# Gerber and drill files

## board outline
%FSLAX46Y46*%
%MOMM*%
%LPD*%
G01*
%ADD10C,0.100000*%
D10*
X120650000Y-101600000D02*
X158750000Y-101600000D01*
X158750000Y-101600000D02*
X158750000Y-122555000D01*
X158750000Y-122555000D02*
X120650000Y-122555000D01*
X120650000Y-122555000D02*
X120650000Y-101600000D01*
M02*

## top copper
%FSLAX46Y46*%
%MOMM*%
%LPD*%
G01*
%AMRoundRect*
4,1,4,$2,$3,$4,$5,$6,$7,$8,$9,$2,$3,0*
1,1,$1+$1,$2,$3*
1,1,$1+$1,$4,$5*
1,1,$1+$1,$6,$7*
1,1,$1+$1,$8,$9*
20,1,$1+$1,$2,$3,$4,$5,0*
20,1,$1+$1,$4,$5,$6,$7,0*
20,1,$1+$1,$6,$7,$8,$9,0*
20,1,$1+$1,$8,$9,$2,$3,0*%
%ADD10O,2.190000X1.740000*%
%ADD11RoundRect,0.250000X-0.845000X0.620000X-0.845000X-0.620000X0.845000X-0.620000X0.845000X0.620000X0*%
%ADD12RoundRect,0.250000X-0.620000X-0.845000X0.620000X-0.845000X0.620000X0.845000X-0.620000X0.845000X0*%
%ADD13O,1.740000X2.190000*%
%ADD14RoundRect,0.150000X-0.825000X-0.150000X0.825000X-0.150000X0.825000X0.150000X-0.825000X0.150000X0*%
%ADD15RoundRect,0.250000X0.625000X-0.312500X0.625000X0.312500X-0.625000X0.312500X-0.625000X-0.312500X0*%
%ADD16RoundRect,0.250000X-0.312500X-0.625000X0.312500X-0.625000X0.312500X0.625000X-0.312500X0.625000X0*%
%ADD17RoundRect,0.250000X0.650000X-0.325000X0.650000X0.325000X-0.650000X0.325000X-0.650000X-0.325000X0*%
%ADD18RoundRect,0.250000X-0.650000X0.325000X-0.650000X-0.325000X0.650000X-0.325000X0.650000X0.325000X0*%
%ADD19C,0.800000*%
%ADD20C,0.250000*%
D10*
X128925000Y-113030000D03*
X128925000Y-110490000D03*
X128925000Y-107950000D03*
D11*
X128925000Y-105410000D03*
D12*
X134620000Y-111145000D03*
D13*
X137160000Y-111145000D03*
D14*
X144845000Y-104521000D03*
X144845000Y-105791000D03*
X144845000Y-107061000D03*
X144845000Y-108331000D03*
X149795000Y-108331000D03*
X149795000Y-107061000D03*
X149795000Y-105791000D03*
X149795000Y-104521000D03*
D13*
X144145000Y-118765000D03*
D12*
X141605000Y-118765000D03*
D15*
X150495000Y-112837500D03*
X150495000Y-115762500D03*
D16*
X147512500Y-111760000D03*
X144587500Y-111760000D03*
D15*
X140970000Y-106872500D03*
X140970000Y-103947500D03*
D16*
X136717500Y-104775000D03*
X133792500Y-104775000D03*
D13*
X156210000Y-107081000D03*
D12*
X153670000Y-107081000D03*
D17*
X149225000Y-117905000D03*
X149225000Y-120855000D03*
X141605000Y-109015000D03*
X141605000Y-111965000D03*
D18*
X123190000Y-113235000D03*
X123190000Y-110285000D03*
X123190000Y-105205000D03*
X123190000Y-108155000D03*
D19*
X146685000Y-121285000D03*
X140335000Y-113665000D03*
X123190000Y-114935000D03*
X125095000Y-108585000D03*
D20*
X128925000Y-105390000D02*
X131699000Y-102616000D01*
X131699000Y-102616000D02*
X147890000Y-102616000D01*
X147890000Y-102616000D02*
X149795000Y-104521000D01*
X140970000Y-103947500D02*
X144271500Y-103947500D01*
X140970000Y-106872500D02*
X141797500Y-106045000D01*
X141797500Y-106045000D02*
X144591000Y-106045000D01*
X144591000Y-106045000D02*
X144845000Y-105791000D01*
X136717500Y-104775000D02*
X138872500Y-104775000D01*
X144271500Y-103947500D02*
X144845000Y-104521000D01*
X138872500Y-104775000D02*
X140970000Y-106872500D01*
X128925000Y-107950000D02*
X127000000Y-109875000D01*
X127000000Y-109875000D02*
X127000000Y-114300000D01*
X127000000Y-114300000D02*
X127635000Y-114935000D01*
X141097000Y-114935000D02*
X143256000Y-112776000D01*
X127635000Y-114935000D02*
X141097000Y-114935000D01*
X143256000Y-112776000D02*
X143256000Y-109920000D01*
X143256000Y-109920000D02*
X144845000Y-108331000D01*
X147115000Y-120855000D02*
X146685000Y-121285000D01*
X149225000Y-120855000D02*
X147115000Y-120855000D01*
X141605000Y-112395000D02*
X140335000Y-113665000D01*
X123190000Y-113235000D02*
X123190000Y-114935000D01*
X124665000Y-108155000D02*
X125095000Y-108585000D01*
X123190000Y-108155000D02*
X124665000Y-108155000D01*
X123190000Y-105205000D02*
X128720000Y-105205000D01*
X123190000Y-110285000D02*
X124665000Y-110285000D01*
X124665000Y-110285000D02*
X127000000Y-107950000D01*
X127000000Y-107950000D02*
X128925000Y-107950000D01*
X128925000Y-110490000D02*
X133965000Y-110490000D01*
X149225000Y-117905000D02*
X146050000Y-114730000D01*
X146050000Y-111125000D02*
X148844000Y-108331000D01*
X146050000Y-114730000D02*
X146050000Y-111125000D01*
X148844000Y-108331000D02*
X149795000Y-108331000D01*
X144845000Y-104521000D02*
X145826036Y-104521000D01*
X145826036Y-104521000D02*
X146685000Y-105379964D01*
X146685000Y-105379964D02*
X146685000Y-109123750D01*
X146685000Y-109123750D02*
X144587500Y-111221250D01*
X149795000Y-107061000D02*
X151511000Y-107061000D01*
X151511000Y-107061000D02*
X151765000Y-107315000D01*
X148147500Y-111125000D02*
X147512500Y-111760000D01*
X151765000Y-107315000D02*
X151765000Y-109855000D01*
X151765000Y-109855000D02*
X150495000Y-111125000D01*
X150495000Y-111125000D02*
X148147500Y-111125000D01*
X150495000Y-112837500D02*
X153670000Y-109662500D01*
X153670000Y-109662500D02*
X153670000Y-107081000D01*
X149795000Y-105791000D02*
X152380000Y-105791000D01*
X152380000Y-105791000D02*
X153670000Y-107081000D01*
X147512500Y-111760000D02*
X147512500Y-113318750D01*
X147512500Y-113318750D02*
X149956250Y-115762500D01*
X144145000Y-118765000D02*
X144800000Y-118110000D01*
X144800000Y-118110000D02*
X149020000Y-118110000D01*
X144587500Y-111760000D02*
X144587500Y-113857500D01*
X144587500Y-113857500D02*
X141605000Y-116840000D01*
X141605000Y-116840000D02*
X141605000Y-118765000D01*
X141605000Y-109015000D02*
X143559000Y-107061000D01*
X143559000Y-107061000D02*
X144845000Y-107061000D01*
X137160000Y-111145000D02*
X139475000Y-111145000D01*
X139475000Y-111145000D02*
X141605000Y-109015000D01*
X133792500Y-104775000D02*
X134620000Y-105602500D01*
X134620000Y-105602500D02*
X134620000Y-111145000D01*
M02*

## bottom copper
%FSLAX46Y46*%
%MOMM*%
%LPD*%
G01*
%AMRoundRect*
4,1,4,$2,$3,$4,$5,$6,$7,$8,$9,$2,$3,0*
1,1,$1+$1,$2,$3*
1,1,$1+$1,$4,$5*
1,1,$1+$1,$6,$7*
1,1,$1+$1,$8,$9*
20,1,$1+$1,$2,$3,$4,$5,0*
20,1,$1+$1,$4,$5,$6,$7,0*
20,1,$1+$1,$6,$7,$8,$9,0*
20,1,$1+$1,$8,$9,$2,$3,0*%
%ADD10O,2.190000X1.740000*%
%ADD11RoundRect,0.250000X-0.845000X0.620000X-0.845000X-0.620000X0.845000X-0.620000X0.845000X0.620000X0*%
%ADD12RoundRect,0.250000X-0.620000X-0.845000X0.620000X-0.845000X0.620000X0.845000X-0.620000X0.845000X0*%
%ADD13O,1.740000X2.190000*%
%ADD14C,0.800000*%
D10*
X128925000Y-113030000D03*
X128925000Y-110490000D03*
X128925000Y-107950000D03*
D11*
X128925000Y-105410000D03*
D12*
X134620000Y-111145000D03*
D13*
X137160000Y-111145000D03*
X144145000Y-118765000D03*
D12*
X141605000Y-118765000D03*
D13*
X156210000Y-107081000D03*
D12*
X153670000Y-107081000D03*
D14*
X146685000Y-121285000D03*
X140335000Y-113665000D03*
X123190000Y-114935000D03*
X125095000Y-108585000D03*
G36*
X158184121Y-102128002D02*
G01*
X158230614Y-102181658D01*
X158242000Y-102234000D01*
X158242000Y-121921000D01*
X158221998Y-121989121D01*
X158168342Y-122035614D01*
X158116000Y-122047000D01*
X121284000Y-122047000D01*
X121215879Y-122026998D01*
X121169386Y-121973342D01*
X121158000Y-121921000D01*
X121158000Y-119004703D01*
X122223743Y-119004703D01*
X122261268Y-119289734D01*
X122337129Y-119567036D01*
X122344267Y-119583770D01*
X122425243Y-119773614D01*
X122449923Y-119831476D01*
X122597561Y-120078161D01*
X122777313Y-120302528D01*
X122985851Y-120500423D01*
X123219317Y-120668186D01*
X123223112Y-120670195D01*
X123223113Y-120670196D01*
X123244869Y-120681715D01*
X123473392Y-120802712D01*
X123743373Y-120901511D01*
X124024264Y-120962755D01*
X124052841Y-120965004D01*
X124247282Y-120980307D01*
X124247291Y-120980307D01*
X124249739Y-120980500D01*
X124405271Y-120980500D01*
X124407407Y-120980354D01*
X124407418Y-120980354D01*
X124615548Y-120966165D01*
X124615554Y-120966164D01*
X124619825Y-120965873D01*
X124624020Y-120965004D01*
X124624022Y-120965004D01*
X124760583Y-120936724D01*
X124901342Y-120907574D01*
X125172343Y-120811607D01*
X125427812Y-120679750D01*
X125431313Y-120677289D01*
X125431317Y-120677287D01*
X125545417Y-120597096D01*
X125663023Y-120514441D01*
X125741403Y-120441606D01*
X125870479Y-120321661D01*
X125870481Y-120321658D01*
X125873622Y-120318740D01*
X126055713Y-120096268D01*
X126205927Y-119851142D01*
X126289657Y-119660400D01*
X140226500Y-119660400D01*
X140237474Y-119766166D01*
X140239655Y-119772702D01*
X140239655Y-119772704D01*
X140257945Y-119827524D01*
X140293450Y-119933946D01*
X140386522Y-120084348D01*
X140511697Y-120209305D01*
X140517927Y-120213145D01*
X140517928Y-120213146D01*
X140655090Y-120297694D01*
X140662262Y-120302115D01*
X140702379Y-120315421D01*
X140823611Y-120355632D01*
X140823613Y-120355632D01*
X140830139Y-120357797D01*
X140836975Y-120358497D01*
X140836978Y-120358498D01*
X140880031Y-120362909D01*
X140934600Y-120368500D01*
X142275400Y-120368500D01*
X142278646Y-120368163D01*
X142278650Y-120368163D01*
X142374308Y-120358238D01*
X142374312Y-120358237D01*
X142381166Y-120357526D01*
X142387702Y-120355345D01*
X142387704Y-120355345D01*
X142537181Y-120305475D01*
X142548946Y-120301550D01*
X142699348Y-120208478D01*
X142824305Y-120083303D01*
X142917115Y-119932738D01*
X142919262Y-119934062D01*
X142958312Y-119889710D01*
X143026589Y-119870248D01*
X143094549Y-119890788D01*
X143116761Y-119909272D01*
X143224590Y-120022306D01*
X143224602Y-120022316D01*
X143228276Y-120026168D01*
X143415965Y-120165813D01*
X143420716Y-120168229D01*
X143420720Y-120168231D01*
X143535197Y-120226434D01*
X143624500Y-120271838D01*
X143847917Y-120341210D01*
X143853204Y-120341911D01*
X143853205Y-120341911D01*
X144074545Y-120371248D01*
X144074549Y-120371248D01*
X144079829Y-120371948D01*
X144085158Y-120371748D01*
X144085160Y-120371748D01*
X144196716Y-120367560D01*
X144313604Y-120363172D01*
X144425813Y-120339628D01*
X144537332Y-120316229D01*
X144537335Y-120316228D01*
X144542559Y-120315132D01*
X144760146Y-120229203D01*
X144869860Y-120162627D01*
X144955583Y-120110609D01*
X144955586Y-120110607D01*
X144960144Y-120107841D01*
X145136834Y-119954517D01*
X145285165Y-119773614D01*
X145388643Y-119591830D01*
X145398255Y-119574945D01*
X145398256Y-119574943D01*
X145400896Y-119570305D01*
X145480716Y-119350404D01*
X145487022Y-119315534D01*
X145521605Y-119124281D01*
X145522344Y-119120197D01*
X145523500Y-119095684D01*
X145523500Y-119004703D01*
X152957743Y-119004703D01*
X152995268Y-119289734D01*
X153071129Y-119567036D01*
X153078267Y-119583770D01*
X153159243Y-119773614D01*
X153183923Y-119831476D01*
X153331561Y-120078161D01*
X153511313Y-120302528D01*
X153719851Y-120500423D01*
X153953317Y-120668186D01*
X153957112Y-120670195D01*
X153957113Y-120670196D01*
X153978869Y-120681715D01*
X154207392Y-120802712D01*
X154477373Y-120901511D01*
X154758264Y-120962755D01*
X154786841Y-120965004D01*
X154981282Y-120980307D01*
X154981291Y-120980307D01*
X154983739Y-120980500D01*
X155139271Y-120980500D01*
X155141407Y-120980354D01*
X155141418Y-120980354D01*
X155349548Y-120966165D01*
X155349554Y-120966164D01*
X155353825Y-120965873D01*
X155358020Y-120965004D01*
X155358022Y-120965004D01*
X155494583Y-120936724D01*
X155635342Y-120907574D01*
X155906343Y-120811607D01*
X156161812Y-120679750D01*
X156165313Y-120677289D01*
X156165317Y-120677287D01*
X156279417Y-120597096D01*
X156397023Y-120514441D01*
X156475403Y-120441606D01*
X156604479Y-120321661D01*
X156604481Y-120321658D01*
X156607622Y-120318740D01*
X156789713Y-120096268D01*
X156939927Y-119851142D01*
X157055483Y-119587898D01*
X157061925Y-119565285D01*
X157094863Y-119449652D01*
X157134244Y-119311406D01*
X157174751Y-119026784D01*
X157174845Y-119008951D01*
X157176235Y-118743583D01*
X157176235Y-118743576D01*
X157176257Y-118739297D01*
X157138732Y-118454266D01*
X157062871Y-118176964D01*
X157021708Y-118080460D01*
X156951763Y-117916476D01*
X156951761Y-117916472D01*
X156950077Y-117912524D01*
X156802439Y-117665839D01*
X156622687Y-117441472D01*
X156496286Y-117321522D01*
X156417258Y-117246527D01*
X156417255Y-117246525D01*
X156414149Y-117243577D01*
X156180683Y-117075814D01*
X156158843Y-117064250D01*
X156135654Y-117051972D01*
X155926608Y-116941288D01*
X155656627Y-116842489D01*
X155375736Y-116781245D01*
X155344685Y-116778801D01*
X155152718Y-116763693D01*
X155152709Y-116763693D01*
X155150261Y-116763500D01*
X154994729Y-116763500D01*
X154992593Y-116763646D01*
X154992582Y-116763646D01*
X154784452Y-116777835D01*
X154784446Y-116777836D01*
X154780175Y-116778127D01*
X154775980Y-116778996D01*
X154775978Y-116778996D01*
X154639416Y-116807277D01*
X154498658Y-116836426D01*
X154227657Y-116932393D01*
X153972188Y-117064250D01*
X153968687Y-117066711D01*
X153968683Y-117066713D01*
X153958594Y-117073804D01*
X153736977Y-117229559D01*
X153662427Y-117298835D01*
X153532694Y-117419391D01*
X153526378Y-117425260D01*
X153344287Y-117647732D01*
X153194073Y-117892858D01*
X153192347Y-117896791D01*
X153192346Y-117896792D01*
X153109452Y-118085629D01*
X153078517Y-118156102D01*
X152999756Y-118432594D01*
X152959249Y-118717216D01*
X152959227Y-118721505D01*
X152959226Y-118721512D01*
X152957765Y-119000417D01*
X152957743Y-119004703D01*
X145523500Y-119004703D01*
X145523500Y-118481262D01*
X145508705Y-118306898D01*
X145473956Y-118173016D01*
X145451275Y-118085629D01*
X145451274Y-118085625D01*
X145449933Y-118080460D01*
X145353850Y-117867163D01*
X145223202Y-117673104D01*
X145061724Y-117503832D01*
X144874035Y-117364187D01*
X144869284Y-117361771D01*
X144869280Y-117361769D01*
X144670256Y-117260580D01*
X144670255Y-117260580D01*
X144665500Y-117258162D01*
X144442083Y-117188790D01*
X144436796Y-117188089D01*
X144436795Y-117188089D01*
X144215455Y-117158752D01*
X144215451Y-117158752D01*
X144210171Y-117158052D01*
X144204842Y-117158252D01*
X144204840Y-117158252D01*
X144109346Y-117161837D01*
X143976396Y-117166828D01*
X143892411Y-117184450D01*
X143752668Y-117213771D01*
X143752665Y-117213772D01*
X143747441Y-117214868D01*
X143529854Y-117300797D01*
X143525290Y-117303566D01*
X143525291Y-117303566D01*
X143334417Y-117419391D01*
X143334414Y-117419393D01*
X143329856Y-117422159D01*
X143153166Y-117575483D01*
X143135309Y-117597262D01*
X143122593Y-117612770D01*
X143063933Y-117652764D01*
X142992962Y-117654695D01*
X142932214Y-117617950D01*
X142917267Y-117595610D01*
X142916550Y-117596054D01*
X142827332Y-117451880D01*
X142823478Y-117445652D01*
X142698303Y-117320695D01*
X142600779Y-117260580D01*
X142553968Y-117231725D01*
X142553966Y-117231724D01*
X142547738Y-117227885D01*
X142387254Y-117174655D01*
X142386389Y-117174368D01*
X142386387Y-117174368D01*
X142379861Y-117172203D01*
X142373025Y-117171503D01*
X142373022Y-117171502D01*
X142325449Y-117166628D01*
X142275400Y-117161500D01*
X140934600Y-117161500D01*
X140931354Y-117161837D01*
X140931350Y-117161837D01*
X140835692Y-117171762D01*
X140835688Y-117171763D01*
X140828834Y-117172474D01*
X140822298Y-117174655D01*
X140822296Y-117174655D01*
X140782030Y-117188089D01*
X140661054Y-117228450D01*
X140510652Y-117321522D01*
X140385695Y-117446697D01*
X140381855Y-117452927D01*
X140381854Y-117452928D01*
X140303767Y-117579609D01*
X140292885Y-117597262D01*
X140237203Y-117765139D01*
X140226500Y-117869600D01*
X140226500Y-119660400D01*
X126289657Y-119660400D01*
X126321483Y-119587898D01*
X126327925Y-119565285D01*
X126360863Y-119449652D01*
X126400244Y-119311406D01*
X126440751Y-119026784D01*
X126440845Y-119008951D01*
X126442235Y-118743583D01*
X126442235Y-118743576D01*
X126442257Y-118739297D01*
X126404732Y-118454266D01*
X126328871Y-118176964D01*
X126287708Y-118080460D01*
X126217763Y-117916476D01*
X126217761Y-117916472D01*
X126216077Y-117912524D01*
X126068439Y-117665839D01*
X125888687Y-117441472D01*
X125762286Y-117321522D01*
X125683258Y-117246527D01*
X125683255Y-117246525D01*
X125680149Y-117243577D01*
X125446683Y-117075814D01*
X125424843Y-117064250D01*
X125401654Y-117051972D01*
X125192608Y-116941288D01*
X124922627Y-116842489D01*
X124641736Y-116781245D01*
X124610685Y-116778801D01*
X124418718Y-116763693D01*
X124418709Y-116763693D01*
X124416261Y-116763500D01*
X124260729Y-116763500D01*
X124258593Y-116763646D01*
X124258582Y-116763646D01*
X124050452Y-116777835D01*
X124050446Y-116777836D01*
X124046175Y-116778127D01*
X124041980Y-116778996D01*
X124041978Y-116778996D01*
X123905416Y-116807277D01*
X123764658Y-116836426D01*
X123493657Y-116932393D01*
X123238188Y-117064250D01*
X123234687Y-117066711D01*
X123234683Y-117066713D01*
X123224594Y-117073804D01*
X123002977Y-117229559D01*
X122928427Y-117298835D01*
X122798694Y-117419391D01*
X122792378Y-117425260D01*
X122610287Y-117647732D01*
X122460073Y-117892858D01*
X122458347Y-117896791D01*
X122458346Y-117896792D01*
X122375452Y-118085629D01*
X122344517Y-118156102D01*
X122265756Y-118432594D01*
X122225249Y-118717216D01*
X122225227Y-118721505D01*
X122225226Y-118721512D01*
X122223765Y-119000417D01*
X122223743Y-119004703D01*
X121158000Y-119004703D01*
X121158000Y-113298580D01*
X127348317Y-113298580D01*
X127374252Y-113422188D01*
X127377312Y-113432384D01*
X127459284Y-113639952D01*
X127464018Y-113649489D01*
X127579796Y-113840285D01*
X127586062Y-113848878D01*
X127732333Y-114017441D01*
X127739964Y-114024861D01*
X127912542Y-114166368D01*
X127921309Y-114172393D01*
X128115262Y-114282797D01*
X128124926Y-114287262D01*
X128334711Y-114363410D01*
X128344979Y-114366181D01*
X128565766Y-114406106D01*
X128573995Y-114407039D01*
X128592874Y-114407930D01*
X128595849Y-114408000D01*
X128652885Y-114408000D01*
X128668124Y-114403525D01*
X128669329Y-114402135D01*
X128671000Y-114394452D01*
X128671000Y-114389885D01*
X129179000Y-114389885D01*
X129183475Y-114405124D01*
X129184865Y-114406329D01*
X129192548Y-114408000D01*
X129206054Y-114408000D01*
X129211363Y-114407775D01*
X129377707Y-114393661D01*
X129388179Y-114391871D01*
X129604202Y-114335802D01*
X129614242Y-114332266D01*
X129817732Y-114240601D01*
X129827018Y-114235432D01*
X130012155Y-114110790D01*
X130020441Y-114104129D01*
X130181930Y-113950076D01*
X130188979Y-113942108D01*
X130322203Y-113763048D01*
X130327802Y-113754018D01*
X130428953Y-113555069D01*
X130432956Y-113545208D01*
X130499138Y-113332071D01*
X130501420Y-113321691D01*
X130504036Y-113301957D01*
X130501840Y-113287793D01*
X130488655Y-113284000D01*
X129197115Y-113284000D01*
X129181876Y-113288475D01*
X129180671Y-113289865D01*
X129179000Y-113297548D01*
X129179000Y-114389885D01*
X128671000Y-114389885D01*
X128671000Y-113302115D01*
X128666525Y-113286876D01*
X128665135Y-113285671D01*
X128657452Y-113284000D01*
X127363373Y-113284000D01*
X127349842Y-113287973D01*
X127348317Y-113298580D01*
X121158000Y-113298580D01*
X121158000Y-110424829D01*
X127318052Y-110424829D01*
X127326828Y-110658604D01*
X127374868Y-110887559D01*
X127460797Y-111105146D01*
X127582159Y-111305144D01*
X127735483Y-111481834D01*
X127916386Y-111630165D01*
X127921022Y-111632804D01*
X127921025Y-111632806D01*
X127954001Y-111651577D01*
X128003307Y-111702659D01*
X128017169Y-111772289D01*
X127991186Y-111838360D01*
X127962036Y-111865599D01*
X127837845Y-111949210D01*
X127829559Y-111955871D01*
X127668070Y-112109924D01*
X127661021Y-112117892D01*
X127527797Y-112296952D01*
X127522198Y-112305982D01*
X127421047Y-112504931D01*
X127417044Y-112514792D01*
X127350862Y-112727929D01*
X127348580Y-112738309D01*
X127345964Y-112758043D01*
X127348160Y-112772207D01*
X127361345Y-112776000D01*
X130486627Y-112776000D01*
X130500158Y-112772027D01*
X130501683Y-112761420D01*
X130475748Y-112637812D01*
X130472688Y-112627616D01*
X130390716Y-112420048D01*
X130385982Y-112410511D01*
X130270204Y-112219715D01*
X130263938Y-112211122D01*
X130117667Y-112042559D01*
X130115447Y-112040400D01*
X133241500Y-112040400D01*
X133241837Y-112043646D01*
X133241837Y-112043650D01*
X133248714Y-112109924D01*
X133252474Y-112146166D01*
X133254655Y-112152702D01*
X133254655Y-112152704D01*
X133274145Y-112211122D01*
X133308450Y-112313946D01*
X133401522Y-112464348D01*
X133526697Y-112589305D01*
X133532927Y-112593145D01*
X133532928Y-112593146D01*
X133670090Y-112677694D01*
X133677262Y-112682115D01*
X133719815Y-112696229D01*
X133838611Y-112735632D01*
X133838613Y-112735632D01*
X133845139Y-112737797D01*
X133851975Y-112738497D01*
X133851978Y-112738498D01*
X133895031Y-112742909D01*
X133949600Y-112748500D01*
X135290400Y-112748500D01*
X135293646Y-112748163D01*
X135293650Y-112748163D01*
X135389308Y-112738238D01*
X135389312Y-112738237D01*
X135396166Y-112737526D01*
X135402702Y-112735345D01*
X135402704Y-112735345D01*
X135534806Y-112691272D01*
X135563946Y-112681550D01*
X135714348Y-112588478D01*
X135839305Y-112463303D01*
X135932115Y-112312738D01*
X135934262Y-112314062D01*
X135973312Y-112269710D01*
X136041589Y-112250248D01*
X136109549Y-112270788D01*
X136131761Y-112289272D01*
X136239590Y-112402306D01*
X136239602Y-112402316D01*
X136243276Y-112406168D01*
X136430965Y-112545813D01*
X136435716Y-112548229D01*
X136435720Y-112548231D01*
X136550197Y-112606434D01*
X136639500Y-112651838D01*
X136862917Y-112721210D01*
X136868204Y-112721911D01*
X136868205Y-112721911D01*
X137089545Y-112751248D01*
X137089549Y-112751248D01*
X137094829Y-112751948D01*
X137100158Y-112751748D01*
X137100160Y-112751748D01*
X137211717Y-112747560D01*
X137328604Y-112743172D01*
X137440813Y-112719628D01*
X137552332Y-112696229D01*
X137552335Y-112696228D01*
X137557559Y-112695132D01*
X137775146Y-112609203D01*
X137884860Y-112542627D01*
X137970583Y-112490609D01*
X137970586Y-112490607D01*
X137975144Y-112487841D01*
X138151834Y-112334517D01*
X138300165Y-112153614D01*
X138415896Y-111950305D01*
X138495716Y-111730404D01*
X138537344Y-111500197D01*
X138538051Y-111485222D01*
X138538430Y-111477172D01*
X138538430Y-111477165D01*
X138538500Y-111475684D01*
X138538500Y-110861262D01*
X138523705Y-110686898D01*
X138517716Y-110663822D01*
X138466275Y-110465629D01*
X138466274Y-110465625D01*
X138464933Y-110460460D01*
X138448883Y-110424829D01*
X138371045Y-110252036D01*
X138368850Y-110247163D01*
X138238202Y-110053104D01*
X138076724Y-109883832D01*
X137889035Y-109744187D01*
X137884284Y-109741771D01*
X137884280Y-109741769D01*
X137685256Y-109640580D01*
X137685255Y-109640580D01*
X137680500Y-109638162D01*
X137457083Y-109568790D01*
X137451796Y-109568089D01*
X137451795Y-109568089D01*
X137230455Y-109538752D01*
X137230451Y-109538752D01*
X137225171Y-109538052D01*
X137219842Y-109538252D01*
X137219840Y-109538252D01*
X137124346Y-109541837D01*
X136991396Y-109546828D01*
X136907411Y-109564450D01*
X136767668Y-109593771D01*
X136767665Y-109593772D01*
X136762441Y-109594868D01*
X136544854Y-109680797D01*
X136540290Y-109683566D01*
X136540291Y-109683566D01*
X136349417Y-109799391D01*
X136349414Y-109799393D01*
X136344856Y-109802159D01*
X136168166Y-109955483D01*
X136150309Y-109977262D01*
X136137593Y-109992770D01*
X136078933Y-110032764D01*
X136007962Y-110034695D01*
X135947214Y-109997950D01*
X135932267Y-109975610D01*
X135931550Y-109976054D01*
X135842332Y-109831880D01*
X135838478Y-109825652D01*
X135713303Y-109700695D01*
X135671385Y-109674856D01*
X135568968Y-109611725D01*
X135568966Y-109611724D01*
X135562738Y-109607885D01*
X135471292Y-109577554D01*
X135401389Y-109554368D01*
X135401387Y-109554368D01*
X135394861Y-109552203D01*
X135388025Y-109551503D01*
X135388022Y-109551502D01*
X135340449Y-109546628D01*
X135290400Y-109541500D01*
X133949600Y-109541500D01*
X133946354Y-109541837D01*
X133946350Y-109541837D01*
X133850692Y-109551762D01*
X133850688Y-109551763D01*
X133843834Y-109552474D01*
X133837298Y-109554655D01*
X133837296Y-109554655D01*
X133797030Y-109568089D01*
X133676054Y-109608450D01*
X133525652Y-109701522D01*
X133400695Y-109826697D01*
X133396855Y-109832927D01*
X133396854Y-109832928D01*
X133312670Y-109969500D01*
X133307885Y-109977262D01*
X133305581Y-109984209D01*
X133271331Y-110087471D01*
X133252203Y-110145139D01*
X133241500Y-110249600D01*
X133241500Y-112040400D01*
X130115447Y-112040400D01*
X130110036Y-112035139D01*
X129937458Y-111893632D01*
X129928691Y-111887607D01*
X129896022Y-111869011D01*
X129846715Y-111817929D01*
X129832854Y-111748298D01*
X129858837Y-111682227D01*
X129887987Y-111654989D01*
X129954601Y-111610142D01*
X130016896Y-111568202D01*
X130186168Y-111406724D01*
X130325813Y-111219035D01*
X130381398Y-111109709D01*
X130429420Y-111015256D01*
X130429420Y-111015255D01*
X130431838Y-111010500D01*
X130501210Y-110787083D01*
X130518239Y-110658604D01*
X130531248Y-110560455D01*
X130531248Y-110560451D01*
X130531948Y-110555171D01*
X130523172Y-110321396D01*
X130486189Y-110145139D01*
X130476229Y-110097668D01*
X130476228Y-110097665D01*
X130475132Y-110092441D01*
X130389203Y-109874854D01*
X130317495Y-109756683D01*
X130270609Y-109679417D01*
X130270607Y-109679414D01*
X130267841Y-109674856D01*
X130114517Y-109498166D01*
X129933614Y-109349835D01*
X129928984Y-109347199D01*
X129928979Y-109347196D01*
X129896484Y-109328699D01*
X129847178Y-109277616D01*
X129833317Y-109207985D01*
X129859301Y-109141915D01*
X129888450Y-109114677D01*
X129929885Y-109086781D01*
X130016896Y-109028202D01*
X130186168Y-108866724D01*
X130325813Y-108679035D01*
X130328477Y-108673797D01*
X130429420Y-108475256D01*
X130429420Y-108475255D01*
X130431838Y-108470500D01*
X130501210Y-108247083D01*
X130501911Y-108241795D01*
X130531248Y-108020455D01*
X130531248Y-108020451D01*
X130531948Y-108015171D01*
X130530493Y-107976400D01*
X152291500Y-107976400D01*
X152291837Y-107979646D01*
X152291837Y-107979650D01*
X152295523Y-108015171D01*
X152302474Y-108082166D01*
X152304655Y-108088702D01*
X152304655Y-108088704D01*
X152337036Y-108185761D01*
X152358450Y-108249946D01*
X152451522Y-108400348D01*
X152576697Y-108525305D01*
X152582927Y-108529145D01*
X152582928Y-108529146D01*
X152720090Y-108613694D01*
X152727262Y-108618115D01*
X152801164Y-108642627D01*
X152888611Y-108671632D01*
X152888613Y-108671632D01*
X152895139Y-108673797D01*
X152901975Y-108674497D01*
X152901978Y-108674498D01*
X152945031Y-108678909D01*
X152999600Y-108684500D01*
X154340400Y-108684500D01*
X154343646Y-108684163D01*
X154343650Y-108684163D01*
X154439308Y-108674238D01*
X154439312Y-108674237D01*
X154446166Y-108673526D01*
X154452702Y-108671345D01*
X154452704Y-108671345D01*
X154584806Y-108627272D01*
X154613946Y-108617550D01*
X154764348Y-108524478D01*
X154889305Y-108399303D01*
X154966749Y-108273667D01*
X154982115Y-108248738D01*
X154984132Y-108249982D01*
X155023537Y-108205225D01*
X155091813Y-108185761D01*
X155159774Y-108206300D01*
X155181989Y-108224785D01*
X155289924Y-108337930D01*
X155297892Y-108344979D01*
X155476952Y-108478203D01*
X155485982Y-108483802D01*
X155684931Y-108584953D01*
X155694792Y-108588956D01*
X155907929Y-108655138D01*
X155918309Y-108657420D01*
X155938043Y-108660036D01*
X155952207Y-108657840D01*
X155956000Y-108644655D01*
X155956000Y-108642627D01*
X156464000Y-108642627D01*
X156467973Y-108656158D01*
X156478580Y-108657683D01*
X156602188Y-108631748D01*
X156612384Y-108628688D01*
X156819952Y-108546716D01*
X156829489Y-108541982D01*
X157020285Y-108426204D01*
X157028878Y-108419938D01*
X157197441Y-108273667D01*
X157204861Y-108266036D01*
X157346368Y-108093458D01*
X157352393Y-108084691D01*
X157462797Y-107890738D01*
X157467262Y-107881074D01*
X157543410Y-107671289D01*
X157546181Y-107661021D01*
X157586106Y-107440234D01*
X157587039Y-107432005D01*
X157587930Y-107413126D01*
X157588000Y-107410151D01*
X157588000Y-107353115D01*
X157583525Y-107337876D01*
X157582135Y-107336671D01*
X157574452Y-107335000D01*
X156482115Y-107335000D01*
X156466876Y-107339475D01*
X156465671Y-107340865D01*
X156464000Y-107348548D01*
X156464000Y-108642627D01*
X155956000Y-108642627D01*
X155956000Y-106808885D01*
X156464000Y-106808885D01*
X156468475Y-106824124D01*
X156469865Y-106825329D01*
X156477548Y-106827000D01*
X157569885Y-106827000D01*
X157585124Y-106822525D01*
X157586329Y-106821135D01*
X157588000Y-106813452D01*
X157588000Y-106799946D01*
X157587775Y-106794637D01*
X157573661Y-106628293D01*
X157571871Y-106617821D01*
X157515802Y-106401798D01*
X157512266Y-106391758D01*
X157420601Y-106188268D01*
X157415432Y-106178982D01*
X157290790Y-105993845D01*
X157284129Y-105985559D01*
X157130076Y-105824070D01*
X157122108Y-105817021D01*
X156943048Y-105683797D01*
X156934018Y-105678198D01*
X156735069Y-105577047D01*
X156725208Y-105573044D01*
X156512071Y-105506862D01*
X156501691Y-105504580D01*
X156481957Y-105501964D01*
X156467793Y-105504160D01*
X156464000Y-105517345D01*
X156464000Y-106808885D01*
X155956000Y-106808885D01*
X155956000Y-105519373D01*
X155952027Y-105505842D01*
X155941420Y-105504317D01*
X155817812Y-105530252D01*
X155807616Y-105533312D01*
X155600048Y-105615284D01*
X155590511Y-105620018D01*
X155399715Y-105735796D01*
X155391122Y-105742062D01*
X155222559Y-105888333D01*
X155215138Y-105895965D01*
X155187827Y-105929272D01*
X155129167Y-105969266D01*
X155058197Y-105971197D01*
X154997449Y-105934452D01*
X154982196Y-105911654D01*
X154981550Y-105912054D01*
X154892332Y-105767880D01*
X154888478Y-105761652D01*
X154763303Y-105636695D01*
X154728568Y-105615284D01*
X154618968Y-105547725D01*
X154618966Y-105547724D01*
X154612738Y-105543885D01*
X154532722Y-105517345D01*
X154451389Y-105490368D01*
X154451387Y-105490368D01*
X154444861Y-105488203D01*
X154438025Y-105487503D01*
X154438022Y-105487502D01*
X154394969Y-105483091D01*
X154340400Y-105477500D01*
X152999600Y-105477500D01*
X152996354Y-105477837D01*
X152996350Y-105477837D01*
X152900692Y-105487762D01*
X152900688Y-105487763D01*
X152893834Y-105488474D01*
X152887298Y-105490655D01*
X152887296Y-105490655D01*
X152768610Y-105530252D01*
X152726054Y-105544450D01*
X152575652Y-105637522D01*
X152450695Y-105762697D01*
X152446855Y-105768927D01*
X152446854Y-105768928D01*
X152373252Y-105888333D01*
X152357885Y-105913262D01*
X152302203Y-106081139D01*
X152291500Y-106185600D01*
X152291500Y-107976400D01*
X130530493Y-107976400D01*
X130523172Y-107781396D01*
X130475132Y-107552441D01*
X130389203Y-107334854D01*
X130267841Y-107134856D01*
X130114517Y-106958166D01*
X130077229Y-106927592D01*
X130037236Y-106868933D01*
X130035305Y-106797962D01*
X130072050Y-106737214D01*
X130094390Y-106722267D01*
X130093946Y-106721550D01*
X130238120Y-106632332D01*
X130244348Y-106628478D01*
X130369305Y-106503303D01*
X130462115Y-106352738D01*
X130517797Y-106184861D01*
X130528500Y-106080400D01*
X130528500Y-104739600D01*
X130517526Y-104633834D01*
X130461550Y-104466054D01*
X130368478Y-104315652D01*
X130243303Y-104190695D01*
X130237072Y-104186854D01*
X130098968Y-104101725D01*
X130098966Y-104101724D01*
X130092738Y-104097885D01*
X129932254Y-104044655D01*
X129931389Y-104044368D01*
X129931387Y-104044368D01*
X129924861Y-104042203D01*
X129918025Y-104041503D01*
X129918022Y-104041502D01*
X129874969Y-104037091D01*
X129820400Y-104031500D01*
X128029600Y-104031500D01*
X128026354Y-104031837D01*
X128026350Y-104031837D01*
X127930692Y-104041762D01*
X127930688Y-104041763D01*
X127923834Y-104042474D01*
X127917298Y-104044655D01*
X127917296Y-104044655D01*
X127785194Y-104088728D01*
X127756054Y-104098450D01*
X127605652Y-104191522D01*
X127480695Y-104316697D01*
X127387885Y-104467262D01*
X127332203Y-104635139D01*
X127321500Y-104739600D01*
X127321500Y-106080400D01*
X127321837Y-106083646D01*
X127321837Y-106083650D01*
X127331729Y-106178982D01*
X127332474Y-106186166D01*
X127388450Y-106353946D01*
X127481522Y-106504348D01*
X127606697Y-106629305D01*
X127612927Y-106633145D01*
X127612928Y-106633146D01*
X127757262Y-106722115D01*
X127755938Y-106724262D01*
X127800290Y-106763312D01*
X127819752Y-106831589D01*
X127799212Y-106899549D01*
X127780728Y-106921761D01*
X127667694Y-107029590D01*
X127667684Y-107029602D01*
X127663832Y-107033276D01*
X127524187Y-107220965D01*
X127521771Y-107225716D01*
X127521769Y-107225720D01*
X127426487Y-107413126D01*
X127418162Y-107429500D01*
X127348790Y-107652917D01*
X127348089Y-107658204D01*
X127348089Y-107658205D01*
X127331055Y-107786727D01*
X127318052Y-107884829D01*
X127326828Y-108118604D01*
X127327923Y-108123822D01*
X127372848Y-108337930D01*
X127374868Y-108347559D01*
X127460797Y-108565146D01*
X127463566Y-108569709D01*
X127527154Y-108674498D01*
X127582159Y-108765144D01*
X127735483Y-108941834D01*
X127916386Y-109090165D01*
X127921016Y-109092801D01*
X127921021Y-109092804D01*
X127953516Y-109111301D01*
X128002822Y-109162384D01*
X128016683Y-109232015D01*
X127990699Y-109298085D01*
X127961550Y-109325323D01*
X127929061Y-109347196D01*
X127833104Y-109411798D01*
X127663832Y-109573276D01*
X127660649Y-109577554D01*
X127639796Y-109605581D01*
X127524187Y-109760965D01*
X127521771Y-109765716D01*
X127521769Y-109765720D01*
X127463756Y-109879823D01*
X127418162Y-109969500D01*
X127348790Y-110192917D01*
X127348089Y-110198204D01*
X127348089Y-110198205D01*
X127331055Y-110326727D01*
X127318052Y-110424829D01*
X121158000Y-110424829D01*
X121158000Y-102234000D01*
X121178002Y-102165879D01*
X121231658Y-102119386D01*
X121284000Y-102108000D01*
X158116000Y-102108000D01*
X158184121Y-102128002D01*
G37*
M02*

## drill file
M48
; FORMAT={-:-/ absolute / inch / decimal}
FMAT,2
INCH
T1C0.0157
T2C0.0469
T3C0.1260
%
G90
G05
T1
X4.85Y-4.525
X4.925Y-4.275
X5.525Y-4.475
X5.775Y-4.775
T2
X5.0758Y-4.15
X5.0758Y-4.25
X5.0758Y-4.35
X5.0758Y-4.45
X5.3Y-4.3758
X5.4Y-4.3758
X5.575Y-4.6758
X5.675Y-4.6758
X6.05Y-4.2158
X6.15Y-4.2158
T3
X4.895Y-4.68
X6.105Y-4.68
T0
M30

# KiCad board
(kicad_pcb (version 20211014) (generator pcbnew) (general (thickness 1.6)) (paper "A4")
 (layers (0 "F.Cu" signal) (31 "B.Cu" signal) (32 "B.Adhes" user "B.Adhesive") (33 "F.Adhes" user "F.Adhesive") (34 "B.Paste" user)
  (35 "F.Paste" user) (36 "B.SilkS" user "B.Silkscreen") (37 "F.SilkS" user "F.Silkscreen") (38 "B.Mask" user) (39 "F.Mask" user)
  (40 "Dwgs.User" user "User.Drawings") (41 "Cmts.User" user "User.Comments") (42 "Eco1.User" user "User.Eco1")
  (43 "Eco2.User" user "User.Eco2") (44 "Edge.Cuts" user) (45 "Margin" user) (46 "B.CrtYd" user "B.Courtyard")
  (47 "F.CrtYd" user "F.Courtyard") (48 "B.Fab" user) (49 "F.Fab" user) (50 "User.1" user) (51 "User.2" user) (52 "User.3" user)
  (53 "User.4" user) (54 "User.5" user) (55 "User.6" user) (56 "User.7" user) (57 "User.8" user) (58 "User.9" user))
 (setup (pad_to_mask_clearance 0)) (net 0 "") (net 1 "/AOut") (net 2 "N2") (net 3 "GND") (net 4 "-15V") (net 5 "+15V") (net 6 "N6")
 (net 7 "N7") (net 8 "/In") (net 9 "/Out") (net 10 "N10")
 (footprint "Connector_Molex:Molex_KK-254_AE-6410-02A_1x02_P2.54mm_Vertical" (layer "F.Cu") (at 141.605 118.765)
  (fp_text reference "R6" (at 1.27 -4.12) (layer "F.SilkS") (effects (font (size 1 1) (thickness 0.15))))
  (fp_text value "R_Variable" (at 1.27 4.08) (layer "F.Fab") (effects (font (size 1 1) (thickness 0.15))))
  (pad "1" thru_hole roundrect (at 0 0) (size 1.74 2.19) (drill 1.19) (layers *.Cu *.Mask) (roundrect_rratio 0.1436781609) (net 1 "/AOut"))
  (pad "2" thru_hole oval (at 2.54 0) (size 1.74 2.19) (drill 1.19) (layers *.Cu *.Mask) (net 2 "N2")))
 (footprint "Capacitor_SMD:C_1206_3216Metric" (layer "F.Cu") (at 149.225 119.38 90)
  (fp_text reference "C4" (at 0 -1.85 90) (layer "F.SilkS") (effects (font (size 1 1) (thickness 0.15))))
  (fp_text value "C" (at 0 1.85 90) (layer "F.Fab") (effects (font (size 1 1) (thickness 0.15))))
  (pad "1" smd roundrect (at -1.475 0 90) (size 1.15 1.8) (layers "F.Cu" "F.Paste" "F.Mask") (roundrect_rratio 0.2173913043) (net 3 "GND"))
  (pad "2" smd roundrect (at 1.475 0 90) (size 1.15 1.8) (layers "F.Cu" "F.Paste" "F.Mask") (roundrect_rratio 0.2173913043) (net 2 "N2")))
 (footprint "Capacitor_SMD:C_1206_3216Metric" (layer "F.Cu") (at 123.19 111.76 -90)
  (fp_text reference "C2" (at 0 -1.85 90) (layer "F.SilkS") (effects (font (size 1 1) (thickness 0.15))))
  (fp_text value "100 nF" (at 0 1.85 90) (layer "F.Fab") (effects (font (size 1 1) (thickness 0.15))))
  (pad "1" smd roundrect (at -1.475 0 270) (size 1.15 1.8) (layers "F.Cu" "F.Paste" "F.Mask") (roundrect_rratio 0.2173913043) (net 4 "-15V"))
  (pad "2" smd roundrect (at 1.475 0 270) (size 1.15 1.8) (layers "F.Cu" "F.Paste" "F.Mask") (roundrect_rratio 0.2173913043) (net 3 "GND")))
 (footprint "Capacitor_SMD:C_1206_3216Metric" (layer "F.Cu") (at 123.19 106.68 -90)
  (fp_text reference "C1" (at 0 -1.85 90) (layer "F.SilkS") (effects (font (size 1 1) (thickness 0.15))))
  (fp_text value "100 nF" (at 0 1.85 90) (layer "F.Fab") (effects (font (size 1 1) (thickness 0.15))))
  (pad "1" smd roundrect (at -1.475 0 270) (size 1.15 1.8) (layers "F.Cu" "F.Paste" "F.Mask") (roundrect_rratio 0.2173913043) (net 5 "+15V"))
  (pad "2" smd roundrect (at 1.475 0 270) (size 1.15 1.8) (layers "F.Cu" "F.Paste" "F.Mask") (roundrect_rratio 0.2173913043) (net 3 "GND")))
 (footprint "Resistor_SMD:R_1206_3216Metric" (layer "F.Cu") (at 146.05 111.76)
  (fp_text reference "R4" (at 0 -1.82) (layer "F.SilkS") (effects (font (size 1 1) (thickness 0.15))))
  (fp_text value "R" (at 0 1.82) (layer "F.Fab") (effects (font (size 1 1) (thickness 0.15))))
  (pad "1" smd roundrect (at -1.4625 0) (size 1.125 1.75) (layers "F.Cu" "F.Paste" "F.Mask") (roundrect_rratio 0.2222222222) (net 1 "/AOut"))
  (pad "2" smd roundrect (at 1.4625 0) (size 1.125 1.75) (layers "F.Cu" "F.Paste" "F.Mask") (roundrect_rratio 0.2222222222) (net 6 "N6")))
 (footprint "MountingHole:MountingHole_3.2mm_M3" (layer "F.Cu") (at 124.333 118.872)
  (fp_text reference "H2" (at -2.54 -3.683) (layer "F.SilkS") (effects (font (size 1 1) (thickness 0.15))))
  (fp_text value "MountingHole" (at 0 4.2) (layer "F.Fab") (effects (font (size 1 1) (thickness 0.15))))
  (pad "" np_thru_hole circle (at 0 0) (size 3.2 3.2) (drill 3.2) (layers *.Cu *.Mask)))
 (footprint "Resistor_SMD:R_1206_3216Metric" (layer "F.Cu") (at 140.97 105.41 90)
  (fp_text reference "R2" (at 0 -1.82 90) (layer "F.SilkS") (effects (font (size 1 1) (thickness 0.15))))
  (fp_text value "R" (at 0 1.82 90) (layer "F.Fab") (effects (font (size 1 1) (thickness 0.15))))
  (pad "1" smd roundrect (at -1.4625 0 90) (size 1.125 1.75) (layers "F.Cu" "F.Paste" "F.Mask") (roundrect_rratio 0.2222222222) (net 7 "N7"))
  (pad "2" smd roundrect (at 1.4625 0 90) (size 1.125 1.75) (layers "F.Cu" "F.Paste" "F.Mask") (roundrect_rratio 0.2222222222)
   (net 1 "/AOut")))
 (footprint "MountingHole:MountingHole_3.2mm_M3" (layer "F.Cu") (at 155.067 118.872)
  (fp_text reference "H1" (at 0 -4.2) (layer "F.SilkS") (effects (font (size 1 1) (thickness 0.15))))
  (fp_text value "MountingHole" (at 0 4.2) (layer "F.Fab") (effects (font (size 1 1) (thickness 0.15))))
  (pad "" np_thru_hole circle (at 0 0) (size 3.2 3.2) (drill 3.2) (layers *.Cu *.Mask)))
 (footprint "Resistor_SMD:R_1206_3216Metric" (layer "F.Cu") (at 135.255 104.775)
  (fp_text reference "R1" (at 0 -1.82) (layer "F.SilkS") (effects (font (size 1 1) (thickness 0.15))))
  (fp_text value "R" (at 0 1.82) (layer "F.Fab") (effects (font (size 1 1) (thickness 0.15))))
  (pad "1" smd roundrect (at -1.4625 0) (size 1.125 1.75) (layers "F.Cu" "F.Paste" "F.Mask") (roundrect_rratio 0.2222222222) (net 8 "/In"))
  (pad "2" smd roundrect (at 1.4625 0) (size 1.125 1.75) (layers "F.Cu" "F.Paste" "F.Mask") (roundrect_rratio 0.2222222222) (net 7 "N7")))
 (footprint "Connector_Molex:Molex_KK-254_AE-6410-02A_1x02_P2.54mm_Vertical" (layer "F.Cu") (at 153.67 107.081)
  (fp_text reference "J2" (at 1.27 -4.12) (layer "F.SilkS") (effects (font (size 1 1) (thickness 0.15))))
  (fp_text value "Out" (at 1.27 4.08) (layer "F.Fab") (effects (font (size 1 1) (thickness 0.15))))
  (pad "1" thru_hole roundrect (at 0 0) (size 1.74 2.19) (drill 1.19) (layers *.Cu *.Mask) (roundrect_rratio 0.1436781609) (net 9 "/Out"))
  (pad "2" thru_hole oval (at 2.54 0) (size 1.74 2.19) (drill 1.19) (layers *.Cu *.Mask) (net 3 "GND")))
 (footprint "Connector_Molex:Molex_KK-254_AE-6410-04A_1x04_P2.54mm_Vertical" (layer "F.Cu") (at 128.925 105.41 -90)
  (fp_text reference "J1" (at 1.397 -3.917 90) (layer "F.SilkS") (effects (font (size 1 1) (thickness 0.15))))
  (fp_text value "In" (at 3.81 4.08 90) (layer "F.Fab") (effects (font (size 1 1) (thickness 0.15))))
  (pad "1" thru_hole roundrect (at 0 0 270) (size 1.74 2.19) (drill 1.19) (layers *.Cu *.Mask) (roundrect_rratio 0.1436781609)
   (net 5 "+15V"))
  (pad "2" thru_hole oval (at 2.54 0 270) (size 1.74 2.19) (drill 1.19) (layers *.Cu *.Mask) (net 4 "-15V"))
  (pad "3" thru_hole oval (at 5.08 0 270) (size 1.74 2.19) (drill 1.19) (layers *.Cu *.Mask) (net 8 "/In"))
  (pad "4" thru_hole oval (at 7.62 0 270) (size 1.74 2.19) (drill 1.19) (layers *.Cu *.Mask) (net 3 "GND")))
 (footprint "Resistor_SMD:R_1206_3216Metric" (layer "F.Cu") (at 150.495 114.3 90)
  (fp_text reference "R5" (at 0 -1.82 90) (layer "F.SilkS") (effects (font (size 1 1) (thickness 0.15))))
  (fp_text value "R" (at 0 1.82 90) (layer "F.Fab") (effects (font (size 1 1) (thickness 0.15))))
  (pad "1" smd roundrect (at -1.4625 0 90) (size 1.125 1.75) (layers "F.Cu" "F.Paste" "F.Mask") (roundrect_rratio 0.2222222222) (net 6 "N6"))
  (pad "2" smd roundrect (at 1.4625 0 90) (size 1.125 1.75) (layers "F.Cu" "F.Paste" "F.Mask") (roundrect_rratio 0.2222222222)
   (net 9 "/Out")))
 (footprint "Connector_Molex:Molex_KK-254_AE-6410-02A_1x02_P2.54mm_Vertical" (layer "F.Cu") (at 134.62 111.145)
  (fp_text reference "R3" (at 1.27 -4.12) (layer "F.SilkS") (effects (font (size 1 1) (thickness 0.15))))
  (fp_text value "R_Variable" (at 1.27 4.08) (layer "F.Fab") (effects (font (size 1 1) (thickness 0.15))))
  (pad "1" thru_hole roundrect (at 0 0) (size 1.74 2.19) (drill 1.19) (layers *.Cu *.Mask) (roundrect_rratio 0.1436781609) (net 8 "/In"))
  (pad "2" thru_hole oval (at 2.54 0) (size 1.74 2.19) (drill 1.19) (layers *.Cu *.Mask) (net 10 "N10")))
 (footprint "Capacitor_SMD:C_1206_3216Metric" (layer "F.Cu") (at 141.605 110.49 90)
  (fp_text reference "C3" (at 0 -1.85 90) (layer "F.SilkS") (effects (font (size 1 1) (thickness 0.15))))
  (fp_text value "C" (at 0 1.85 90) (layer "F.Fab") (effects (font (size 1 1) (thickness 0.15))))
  (pad "1" smd roundrect (at -1.475 0 90) (size 1.15 1.8) (layers "F.Cu" "F.Paste" "F.Mask") (roundrect_rratio 0.2173913043) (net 3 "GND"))
  (pad "2" smd roundrect (at 1.475 0 90) (size 1.15 1.8) (layers "F.Cu" "F.Paste" "F.Mask") (roundrect_rratio 0.2173913043) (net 10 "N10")))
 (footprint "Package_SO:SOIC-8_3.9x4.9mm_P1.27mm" (layer "F.Cu") (at 147.32 106.426)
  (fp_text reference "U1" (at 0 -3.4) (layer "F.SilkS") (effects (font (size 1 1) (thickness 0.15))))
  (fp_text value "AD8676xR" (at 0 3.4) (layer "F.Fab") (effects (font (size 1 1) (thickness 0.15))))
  (pad "1" smd roundrect (at -2.475 -1.905) (size 1.95 0.6) (layers "F.Cu" "F.Paste" "F.Mask") (roundrect_rratio 0.25) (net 1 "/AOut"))
  (pad "2" smd roundrect (at -2.475 -0.635) (size 1.95 0.6) (layers "F.Cu" "F.Paste" "F.Mask") (roundrect_rratio 0.25) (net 7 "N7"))
  (pad "3" smd roundrect (at -2.475 0.635) (size 1.95 0.6) (layers "F.Cu" "F.Paste" "F.Mask") (roundrect_rratio 0.25) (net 10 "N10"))
  (pad "4" smd roundrect (at -2.475 1.905) (size 1.95 0.6) (layers "F.Cu" "F.Paste" "F.Mask") (roundrect_rratio 0.25) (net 4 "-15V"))
  (pad "5" smd roundrect (at 2.475 1.905) (size 1.95 0.6) (layers "F.Cu" "F.Paste" "F.Mask") (roundrect_rratio 0.25) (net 2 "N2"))
  (pad "6" smd roundrect (at 2.475 0.635) (size 1.95 0.6) (layers "F.Cu" "F.Paste" "F.Mask") (roundrect_rratio 0.25) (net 6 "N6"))
  (pad "7" smd roundrect (at 2.475 -0.635) (size 1.95 0.6) (layers "F.Cu" "F.Paste" "F.Mask") (roundrect_rratio 0.25) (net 9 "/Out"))
  (pad "8" smd roundrect (at 2.475 -1.905) (size 1.95 0.6) (layers "F.Cu" "F.Paste" "F.Mask") (roundrect_rratio 0.25) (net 5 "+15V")))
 (gr_rect (start 120.65 101.6) (end 158.75 122.555) (layer "Edge.Cuts") (width 0.1) (fill none))
 (segment (start 131.699 102.616) (end 147.89 102.616) (width 0.25) (layer "F.Cu") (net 5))
 (segment (start 123.19 105.205) (end 128.72 105.205) (width 0.25) (layer "F.Cu") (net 5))
 (segment (start 128.925 105.39) (end 131.699 102.616) (width 0.25) (layer "F.Cu") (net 5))
 (segment (start 147.89 102.616) (end 149.795 104.521) (width 0.25) (layer "F.Cu") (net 5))
 (segment (start 123.19 113.235) (end 123.19 114.935) (width 0.25) (layer "F.Cu") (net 3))
 (segment (start 149.225 120.855) (end 147.115 120.855) (width 0.25) (layer "F.Cu") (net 3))
 (segment (start 141.605 112.395) (end 140.335 113.665) (width 0.25) (layer "F.Cu") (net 3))
 (segment (start 124.665 108.155) (end 125.095 108.585) (width 0.25) (layer "F.Cu") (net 3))
 (segment (start 147.115 120.855) (end 146.685 121.285) (width 0.25) (layer "F.Cu") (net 3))
 (segment (start 123.19 108.155) (end 124.665 108.155) (width 0.25) (layer "F.Cu") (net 3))
 (via (at 140.335 113.665) (size 0.8) (drill 0.4) (layers "F.Cu" "B.Cu") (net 3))
 (via (at 125.095 108.585) (size 0.8) (drill 0.4) (layers "F.Cu" "B.Cu") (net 3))
 (via (at 123.19 114.935) (size 0.8) (drill 0.4) (layers "F.Cu" "B.Cu") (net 3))
 (via (at 146.685 121.285) (size 0.8) (drill 0.4) (layers "F.Cu" "B.Cu") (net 3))
 (segment (start 123.19 110.285) (end 124.665 110.285) (width 0.25) (layer "F.Cu") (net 4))
 (segment (start 127.635 114.935) (end 141.097 114.935) (width 0.25) (layer "F.Cu") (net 4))
 (segment (start 143.256 112.776) (end 143.256 109.92) (width 0.25) (layer "F.Cu") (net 4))
 (segment (start 127 107.95) (end 128.925 107.95) (width 0.25) (layer "F.Cu") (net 4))
 (segment (start 143.256 109.92) (end 144.845 108.331) (width 0.25) (layer "F.Cu") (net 4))
 (segment (start 127 114.3) (end 127.635 114.935) (width 0.25) (layer "F.Cu") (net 4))
 (segment (start 127 109.875) (end 127 114.3) (width 0.25) (layer "F.Cu") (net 4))
 (segment (start 124.665 110.285) (end 127 107.95) (width 0.25) (layer "F.Cu") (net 4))
 (segment (start 128.925 107.95) (end 127 109.875) (width 0.25) (layer "F.Cu") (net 4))
 (segment (start 141.097 114.935) (end 143.256 112.776) (width 0.25) (layer "F.Cu") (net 4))
 (segment (start 133.7925 104.775) (end 134.62 105.6025) (width 0.25) (layer "F.Cu") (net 8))
 (segment (start 128.925 110.49) (end 133.965 110.49) (width 0.25) (layer "F.Cu") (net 8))
 (segment (start 134.62 105.6025) (end 134.62 111.145) (width 0.25) (layer "F.Cu") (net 8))
 (segment (start 150.495 112.8375) (end 153.67 109.6625) (width 0.25) (layer "F.Cu") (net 9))
 (segment (start 153.67 109.6625) (end 153.67 107.081) (width 0.25) (layer "F.Cu") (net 9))
 (segment (start 152.38 105.791) (end 153.67 107.081) (width 0.25) (layer "F.Cu") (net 9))
 (segment (start 149.795 105.791) (end 152.38 105.791) (width 0.25) (layer "F.Cu") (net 9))
 (segment (start 136.7175 104.775) (end 138.8725 104.775) (width 0.25) (layer "F.Cu") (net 7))
 (segment (start 141.7975 106.045) (end 144.591 106.045) (width 0.25) (layer "F.Cu") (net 7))
 (segment (start 140.97 106.8725) (end 141.7975 106.045) (width 0.25) (layer "F.Cu") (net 7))
 (segment (start 138.8725 104.775) (end 140.97 106.8725) (width 0.25) (layer "F.Cu") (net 7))
 (segment (start 144.591 106.045) (end 144.845 105.791) (width 0.25) (layer "F.Cu") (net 7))
 (segment (start 149.795 107.061) (end 151.511 107.061) (width 0.25) (layer "F.Cu") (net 6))
 (segment (start 151.765 107.315) (end 151.765 109.855) (width 0.25) (layer "F.Cu") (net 6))
 (segment (start 151.511 107.061) (end 151.765 107.315) (width 0.25) (layer "F.Cu") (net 6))
 (segment (start 148.1475 111.125) (end 147.5125 111.76) (width 0.25) (layer "F.Cu") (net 6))
 (segment (start 151.765 109.855) (end 150.495 111.125) (width 0.25) (layer "F.Cu") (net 6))
 (segment (start 147.5125 113.31875) (end 149.95625 115.7625) (width 0.25) (layer "F.Cu") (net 6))
 (segment (start 150.495 111.125) (end 148.1475 111.125) (width 0.25) (layer "F.Cu") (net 6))
 (segment (start 147.5125 111.76) (end 147.5125 113.31875) (width 0.25) (layer "F.Cu") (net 6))
 (segment (start 146.685 109.12375) (end 144.5875 111.22125) (width 0.25) (layer "F.Cu") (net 1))
 (segment (start 144.845 104.521) (end 145.826036 104.521) (width 0.25) (layer "F.Cu") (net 1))
 (segment (start 140.97 103.9475) (end 144.2715 103.9475) (width 0.25) (layer "F.Cu") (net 1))
 (segment (start 144.2715 103.9475) (end 144.845 104.521) (width 0.25) (layer "F.Cu") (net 1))
 (segment (start 141.605 116.84) (end 141.605 118.765) (width 0.25) (layer "F.Cu") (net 1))
 (segment (start 145.826036 104.521) (end 146.685 105.379964) (width 0.25) (layer "F.Cu") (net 1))
 (segment (start 146.685 105.379964) (end 146.685 109.12375) (width 0.25) (layer "F.Cu") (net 1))
 (segment (start 144.5875 111.76) (end 144.5875 113.8575) (width 0.25) (layer "F.Cu") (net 1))
 (segment (start 144.5875 113.8575) (end 141.605 116.84) (width 0.25) (layer "F.Cu") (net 1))
 (segment (start 139.475 111.145) (end 141.605 109.015) (width 0.25) (layer "F.Cu") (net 10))
 (segment (start 141.605 109.015) (end 143.559 107.061) (width 0.25) (layer "F.Cu") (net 10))
 (segment (start 143.559 107.061) (end 144.845 107.061) (width 0.25) (layer "F.Cu") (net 10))
 (segment (start 137.16 111.145) (end 139.475 111.145) (width 0.25) (layer "F.Cu") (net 10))
 (segment (start 146.05 111.125) (end 148.844 108.331) (width 0.25) (layer "F.Cu") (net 2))
 (segment (start 146.05 114.73) (end 146.05 111.125) (width 0.25) (layer "F.Cu") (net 2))
 (segment (start 148.844 108.331) (end 149.795 108.331) (width 0.25) (layer "F.Cu") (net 2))
 (segment (start 144.8 118.11) (end 149.02 118.11) (width 0.25) (layer "F.Cu") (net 2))
 (segment (start 149.225 117.905) (end 146.05 114.73) (width 0.25) (layer "F.Cu") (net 2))
 (segment (start 144.145 118.765) (end 144.8 118.11) (width 0.25) (layer "F.Cu") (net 2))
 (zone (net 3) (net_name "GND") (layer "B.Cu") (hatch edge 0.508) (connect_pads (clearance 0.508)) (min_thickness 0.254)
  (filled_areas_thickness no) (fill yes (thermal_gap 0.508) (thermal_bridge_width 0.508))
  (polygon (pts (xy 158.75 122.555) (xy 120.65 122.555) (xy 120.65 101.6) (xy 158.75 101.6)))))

